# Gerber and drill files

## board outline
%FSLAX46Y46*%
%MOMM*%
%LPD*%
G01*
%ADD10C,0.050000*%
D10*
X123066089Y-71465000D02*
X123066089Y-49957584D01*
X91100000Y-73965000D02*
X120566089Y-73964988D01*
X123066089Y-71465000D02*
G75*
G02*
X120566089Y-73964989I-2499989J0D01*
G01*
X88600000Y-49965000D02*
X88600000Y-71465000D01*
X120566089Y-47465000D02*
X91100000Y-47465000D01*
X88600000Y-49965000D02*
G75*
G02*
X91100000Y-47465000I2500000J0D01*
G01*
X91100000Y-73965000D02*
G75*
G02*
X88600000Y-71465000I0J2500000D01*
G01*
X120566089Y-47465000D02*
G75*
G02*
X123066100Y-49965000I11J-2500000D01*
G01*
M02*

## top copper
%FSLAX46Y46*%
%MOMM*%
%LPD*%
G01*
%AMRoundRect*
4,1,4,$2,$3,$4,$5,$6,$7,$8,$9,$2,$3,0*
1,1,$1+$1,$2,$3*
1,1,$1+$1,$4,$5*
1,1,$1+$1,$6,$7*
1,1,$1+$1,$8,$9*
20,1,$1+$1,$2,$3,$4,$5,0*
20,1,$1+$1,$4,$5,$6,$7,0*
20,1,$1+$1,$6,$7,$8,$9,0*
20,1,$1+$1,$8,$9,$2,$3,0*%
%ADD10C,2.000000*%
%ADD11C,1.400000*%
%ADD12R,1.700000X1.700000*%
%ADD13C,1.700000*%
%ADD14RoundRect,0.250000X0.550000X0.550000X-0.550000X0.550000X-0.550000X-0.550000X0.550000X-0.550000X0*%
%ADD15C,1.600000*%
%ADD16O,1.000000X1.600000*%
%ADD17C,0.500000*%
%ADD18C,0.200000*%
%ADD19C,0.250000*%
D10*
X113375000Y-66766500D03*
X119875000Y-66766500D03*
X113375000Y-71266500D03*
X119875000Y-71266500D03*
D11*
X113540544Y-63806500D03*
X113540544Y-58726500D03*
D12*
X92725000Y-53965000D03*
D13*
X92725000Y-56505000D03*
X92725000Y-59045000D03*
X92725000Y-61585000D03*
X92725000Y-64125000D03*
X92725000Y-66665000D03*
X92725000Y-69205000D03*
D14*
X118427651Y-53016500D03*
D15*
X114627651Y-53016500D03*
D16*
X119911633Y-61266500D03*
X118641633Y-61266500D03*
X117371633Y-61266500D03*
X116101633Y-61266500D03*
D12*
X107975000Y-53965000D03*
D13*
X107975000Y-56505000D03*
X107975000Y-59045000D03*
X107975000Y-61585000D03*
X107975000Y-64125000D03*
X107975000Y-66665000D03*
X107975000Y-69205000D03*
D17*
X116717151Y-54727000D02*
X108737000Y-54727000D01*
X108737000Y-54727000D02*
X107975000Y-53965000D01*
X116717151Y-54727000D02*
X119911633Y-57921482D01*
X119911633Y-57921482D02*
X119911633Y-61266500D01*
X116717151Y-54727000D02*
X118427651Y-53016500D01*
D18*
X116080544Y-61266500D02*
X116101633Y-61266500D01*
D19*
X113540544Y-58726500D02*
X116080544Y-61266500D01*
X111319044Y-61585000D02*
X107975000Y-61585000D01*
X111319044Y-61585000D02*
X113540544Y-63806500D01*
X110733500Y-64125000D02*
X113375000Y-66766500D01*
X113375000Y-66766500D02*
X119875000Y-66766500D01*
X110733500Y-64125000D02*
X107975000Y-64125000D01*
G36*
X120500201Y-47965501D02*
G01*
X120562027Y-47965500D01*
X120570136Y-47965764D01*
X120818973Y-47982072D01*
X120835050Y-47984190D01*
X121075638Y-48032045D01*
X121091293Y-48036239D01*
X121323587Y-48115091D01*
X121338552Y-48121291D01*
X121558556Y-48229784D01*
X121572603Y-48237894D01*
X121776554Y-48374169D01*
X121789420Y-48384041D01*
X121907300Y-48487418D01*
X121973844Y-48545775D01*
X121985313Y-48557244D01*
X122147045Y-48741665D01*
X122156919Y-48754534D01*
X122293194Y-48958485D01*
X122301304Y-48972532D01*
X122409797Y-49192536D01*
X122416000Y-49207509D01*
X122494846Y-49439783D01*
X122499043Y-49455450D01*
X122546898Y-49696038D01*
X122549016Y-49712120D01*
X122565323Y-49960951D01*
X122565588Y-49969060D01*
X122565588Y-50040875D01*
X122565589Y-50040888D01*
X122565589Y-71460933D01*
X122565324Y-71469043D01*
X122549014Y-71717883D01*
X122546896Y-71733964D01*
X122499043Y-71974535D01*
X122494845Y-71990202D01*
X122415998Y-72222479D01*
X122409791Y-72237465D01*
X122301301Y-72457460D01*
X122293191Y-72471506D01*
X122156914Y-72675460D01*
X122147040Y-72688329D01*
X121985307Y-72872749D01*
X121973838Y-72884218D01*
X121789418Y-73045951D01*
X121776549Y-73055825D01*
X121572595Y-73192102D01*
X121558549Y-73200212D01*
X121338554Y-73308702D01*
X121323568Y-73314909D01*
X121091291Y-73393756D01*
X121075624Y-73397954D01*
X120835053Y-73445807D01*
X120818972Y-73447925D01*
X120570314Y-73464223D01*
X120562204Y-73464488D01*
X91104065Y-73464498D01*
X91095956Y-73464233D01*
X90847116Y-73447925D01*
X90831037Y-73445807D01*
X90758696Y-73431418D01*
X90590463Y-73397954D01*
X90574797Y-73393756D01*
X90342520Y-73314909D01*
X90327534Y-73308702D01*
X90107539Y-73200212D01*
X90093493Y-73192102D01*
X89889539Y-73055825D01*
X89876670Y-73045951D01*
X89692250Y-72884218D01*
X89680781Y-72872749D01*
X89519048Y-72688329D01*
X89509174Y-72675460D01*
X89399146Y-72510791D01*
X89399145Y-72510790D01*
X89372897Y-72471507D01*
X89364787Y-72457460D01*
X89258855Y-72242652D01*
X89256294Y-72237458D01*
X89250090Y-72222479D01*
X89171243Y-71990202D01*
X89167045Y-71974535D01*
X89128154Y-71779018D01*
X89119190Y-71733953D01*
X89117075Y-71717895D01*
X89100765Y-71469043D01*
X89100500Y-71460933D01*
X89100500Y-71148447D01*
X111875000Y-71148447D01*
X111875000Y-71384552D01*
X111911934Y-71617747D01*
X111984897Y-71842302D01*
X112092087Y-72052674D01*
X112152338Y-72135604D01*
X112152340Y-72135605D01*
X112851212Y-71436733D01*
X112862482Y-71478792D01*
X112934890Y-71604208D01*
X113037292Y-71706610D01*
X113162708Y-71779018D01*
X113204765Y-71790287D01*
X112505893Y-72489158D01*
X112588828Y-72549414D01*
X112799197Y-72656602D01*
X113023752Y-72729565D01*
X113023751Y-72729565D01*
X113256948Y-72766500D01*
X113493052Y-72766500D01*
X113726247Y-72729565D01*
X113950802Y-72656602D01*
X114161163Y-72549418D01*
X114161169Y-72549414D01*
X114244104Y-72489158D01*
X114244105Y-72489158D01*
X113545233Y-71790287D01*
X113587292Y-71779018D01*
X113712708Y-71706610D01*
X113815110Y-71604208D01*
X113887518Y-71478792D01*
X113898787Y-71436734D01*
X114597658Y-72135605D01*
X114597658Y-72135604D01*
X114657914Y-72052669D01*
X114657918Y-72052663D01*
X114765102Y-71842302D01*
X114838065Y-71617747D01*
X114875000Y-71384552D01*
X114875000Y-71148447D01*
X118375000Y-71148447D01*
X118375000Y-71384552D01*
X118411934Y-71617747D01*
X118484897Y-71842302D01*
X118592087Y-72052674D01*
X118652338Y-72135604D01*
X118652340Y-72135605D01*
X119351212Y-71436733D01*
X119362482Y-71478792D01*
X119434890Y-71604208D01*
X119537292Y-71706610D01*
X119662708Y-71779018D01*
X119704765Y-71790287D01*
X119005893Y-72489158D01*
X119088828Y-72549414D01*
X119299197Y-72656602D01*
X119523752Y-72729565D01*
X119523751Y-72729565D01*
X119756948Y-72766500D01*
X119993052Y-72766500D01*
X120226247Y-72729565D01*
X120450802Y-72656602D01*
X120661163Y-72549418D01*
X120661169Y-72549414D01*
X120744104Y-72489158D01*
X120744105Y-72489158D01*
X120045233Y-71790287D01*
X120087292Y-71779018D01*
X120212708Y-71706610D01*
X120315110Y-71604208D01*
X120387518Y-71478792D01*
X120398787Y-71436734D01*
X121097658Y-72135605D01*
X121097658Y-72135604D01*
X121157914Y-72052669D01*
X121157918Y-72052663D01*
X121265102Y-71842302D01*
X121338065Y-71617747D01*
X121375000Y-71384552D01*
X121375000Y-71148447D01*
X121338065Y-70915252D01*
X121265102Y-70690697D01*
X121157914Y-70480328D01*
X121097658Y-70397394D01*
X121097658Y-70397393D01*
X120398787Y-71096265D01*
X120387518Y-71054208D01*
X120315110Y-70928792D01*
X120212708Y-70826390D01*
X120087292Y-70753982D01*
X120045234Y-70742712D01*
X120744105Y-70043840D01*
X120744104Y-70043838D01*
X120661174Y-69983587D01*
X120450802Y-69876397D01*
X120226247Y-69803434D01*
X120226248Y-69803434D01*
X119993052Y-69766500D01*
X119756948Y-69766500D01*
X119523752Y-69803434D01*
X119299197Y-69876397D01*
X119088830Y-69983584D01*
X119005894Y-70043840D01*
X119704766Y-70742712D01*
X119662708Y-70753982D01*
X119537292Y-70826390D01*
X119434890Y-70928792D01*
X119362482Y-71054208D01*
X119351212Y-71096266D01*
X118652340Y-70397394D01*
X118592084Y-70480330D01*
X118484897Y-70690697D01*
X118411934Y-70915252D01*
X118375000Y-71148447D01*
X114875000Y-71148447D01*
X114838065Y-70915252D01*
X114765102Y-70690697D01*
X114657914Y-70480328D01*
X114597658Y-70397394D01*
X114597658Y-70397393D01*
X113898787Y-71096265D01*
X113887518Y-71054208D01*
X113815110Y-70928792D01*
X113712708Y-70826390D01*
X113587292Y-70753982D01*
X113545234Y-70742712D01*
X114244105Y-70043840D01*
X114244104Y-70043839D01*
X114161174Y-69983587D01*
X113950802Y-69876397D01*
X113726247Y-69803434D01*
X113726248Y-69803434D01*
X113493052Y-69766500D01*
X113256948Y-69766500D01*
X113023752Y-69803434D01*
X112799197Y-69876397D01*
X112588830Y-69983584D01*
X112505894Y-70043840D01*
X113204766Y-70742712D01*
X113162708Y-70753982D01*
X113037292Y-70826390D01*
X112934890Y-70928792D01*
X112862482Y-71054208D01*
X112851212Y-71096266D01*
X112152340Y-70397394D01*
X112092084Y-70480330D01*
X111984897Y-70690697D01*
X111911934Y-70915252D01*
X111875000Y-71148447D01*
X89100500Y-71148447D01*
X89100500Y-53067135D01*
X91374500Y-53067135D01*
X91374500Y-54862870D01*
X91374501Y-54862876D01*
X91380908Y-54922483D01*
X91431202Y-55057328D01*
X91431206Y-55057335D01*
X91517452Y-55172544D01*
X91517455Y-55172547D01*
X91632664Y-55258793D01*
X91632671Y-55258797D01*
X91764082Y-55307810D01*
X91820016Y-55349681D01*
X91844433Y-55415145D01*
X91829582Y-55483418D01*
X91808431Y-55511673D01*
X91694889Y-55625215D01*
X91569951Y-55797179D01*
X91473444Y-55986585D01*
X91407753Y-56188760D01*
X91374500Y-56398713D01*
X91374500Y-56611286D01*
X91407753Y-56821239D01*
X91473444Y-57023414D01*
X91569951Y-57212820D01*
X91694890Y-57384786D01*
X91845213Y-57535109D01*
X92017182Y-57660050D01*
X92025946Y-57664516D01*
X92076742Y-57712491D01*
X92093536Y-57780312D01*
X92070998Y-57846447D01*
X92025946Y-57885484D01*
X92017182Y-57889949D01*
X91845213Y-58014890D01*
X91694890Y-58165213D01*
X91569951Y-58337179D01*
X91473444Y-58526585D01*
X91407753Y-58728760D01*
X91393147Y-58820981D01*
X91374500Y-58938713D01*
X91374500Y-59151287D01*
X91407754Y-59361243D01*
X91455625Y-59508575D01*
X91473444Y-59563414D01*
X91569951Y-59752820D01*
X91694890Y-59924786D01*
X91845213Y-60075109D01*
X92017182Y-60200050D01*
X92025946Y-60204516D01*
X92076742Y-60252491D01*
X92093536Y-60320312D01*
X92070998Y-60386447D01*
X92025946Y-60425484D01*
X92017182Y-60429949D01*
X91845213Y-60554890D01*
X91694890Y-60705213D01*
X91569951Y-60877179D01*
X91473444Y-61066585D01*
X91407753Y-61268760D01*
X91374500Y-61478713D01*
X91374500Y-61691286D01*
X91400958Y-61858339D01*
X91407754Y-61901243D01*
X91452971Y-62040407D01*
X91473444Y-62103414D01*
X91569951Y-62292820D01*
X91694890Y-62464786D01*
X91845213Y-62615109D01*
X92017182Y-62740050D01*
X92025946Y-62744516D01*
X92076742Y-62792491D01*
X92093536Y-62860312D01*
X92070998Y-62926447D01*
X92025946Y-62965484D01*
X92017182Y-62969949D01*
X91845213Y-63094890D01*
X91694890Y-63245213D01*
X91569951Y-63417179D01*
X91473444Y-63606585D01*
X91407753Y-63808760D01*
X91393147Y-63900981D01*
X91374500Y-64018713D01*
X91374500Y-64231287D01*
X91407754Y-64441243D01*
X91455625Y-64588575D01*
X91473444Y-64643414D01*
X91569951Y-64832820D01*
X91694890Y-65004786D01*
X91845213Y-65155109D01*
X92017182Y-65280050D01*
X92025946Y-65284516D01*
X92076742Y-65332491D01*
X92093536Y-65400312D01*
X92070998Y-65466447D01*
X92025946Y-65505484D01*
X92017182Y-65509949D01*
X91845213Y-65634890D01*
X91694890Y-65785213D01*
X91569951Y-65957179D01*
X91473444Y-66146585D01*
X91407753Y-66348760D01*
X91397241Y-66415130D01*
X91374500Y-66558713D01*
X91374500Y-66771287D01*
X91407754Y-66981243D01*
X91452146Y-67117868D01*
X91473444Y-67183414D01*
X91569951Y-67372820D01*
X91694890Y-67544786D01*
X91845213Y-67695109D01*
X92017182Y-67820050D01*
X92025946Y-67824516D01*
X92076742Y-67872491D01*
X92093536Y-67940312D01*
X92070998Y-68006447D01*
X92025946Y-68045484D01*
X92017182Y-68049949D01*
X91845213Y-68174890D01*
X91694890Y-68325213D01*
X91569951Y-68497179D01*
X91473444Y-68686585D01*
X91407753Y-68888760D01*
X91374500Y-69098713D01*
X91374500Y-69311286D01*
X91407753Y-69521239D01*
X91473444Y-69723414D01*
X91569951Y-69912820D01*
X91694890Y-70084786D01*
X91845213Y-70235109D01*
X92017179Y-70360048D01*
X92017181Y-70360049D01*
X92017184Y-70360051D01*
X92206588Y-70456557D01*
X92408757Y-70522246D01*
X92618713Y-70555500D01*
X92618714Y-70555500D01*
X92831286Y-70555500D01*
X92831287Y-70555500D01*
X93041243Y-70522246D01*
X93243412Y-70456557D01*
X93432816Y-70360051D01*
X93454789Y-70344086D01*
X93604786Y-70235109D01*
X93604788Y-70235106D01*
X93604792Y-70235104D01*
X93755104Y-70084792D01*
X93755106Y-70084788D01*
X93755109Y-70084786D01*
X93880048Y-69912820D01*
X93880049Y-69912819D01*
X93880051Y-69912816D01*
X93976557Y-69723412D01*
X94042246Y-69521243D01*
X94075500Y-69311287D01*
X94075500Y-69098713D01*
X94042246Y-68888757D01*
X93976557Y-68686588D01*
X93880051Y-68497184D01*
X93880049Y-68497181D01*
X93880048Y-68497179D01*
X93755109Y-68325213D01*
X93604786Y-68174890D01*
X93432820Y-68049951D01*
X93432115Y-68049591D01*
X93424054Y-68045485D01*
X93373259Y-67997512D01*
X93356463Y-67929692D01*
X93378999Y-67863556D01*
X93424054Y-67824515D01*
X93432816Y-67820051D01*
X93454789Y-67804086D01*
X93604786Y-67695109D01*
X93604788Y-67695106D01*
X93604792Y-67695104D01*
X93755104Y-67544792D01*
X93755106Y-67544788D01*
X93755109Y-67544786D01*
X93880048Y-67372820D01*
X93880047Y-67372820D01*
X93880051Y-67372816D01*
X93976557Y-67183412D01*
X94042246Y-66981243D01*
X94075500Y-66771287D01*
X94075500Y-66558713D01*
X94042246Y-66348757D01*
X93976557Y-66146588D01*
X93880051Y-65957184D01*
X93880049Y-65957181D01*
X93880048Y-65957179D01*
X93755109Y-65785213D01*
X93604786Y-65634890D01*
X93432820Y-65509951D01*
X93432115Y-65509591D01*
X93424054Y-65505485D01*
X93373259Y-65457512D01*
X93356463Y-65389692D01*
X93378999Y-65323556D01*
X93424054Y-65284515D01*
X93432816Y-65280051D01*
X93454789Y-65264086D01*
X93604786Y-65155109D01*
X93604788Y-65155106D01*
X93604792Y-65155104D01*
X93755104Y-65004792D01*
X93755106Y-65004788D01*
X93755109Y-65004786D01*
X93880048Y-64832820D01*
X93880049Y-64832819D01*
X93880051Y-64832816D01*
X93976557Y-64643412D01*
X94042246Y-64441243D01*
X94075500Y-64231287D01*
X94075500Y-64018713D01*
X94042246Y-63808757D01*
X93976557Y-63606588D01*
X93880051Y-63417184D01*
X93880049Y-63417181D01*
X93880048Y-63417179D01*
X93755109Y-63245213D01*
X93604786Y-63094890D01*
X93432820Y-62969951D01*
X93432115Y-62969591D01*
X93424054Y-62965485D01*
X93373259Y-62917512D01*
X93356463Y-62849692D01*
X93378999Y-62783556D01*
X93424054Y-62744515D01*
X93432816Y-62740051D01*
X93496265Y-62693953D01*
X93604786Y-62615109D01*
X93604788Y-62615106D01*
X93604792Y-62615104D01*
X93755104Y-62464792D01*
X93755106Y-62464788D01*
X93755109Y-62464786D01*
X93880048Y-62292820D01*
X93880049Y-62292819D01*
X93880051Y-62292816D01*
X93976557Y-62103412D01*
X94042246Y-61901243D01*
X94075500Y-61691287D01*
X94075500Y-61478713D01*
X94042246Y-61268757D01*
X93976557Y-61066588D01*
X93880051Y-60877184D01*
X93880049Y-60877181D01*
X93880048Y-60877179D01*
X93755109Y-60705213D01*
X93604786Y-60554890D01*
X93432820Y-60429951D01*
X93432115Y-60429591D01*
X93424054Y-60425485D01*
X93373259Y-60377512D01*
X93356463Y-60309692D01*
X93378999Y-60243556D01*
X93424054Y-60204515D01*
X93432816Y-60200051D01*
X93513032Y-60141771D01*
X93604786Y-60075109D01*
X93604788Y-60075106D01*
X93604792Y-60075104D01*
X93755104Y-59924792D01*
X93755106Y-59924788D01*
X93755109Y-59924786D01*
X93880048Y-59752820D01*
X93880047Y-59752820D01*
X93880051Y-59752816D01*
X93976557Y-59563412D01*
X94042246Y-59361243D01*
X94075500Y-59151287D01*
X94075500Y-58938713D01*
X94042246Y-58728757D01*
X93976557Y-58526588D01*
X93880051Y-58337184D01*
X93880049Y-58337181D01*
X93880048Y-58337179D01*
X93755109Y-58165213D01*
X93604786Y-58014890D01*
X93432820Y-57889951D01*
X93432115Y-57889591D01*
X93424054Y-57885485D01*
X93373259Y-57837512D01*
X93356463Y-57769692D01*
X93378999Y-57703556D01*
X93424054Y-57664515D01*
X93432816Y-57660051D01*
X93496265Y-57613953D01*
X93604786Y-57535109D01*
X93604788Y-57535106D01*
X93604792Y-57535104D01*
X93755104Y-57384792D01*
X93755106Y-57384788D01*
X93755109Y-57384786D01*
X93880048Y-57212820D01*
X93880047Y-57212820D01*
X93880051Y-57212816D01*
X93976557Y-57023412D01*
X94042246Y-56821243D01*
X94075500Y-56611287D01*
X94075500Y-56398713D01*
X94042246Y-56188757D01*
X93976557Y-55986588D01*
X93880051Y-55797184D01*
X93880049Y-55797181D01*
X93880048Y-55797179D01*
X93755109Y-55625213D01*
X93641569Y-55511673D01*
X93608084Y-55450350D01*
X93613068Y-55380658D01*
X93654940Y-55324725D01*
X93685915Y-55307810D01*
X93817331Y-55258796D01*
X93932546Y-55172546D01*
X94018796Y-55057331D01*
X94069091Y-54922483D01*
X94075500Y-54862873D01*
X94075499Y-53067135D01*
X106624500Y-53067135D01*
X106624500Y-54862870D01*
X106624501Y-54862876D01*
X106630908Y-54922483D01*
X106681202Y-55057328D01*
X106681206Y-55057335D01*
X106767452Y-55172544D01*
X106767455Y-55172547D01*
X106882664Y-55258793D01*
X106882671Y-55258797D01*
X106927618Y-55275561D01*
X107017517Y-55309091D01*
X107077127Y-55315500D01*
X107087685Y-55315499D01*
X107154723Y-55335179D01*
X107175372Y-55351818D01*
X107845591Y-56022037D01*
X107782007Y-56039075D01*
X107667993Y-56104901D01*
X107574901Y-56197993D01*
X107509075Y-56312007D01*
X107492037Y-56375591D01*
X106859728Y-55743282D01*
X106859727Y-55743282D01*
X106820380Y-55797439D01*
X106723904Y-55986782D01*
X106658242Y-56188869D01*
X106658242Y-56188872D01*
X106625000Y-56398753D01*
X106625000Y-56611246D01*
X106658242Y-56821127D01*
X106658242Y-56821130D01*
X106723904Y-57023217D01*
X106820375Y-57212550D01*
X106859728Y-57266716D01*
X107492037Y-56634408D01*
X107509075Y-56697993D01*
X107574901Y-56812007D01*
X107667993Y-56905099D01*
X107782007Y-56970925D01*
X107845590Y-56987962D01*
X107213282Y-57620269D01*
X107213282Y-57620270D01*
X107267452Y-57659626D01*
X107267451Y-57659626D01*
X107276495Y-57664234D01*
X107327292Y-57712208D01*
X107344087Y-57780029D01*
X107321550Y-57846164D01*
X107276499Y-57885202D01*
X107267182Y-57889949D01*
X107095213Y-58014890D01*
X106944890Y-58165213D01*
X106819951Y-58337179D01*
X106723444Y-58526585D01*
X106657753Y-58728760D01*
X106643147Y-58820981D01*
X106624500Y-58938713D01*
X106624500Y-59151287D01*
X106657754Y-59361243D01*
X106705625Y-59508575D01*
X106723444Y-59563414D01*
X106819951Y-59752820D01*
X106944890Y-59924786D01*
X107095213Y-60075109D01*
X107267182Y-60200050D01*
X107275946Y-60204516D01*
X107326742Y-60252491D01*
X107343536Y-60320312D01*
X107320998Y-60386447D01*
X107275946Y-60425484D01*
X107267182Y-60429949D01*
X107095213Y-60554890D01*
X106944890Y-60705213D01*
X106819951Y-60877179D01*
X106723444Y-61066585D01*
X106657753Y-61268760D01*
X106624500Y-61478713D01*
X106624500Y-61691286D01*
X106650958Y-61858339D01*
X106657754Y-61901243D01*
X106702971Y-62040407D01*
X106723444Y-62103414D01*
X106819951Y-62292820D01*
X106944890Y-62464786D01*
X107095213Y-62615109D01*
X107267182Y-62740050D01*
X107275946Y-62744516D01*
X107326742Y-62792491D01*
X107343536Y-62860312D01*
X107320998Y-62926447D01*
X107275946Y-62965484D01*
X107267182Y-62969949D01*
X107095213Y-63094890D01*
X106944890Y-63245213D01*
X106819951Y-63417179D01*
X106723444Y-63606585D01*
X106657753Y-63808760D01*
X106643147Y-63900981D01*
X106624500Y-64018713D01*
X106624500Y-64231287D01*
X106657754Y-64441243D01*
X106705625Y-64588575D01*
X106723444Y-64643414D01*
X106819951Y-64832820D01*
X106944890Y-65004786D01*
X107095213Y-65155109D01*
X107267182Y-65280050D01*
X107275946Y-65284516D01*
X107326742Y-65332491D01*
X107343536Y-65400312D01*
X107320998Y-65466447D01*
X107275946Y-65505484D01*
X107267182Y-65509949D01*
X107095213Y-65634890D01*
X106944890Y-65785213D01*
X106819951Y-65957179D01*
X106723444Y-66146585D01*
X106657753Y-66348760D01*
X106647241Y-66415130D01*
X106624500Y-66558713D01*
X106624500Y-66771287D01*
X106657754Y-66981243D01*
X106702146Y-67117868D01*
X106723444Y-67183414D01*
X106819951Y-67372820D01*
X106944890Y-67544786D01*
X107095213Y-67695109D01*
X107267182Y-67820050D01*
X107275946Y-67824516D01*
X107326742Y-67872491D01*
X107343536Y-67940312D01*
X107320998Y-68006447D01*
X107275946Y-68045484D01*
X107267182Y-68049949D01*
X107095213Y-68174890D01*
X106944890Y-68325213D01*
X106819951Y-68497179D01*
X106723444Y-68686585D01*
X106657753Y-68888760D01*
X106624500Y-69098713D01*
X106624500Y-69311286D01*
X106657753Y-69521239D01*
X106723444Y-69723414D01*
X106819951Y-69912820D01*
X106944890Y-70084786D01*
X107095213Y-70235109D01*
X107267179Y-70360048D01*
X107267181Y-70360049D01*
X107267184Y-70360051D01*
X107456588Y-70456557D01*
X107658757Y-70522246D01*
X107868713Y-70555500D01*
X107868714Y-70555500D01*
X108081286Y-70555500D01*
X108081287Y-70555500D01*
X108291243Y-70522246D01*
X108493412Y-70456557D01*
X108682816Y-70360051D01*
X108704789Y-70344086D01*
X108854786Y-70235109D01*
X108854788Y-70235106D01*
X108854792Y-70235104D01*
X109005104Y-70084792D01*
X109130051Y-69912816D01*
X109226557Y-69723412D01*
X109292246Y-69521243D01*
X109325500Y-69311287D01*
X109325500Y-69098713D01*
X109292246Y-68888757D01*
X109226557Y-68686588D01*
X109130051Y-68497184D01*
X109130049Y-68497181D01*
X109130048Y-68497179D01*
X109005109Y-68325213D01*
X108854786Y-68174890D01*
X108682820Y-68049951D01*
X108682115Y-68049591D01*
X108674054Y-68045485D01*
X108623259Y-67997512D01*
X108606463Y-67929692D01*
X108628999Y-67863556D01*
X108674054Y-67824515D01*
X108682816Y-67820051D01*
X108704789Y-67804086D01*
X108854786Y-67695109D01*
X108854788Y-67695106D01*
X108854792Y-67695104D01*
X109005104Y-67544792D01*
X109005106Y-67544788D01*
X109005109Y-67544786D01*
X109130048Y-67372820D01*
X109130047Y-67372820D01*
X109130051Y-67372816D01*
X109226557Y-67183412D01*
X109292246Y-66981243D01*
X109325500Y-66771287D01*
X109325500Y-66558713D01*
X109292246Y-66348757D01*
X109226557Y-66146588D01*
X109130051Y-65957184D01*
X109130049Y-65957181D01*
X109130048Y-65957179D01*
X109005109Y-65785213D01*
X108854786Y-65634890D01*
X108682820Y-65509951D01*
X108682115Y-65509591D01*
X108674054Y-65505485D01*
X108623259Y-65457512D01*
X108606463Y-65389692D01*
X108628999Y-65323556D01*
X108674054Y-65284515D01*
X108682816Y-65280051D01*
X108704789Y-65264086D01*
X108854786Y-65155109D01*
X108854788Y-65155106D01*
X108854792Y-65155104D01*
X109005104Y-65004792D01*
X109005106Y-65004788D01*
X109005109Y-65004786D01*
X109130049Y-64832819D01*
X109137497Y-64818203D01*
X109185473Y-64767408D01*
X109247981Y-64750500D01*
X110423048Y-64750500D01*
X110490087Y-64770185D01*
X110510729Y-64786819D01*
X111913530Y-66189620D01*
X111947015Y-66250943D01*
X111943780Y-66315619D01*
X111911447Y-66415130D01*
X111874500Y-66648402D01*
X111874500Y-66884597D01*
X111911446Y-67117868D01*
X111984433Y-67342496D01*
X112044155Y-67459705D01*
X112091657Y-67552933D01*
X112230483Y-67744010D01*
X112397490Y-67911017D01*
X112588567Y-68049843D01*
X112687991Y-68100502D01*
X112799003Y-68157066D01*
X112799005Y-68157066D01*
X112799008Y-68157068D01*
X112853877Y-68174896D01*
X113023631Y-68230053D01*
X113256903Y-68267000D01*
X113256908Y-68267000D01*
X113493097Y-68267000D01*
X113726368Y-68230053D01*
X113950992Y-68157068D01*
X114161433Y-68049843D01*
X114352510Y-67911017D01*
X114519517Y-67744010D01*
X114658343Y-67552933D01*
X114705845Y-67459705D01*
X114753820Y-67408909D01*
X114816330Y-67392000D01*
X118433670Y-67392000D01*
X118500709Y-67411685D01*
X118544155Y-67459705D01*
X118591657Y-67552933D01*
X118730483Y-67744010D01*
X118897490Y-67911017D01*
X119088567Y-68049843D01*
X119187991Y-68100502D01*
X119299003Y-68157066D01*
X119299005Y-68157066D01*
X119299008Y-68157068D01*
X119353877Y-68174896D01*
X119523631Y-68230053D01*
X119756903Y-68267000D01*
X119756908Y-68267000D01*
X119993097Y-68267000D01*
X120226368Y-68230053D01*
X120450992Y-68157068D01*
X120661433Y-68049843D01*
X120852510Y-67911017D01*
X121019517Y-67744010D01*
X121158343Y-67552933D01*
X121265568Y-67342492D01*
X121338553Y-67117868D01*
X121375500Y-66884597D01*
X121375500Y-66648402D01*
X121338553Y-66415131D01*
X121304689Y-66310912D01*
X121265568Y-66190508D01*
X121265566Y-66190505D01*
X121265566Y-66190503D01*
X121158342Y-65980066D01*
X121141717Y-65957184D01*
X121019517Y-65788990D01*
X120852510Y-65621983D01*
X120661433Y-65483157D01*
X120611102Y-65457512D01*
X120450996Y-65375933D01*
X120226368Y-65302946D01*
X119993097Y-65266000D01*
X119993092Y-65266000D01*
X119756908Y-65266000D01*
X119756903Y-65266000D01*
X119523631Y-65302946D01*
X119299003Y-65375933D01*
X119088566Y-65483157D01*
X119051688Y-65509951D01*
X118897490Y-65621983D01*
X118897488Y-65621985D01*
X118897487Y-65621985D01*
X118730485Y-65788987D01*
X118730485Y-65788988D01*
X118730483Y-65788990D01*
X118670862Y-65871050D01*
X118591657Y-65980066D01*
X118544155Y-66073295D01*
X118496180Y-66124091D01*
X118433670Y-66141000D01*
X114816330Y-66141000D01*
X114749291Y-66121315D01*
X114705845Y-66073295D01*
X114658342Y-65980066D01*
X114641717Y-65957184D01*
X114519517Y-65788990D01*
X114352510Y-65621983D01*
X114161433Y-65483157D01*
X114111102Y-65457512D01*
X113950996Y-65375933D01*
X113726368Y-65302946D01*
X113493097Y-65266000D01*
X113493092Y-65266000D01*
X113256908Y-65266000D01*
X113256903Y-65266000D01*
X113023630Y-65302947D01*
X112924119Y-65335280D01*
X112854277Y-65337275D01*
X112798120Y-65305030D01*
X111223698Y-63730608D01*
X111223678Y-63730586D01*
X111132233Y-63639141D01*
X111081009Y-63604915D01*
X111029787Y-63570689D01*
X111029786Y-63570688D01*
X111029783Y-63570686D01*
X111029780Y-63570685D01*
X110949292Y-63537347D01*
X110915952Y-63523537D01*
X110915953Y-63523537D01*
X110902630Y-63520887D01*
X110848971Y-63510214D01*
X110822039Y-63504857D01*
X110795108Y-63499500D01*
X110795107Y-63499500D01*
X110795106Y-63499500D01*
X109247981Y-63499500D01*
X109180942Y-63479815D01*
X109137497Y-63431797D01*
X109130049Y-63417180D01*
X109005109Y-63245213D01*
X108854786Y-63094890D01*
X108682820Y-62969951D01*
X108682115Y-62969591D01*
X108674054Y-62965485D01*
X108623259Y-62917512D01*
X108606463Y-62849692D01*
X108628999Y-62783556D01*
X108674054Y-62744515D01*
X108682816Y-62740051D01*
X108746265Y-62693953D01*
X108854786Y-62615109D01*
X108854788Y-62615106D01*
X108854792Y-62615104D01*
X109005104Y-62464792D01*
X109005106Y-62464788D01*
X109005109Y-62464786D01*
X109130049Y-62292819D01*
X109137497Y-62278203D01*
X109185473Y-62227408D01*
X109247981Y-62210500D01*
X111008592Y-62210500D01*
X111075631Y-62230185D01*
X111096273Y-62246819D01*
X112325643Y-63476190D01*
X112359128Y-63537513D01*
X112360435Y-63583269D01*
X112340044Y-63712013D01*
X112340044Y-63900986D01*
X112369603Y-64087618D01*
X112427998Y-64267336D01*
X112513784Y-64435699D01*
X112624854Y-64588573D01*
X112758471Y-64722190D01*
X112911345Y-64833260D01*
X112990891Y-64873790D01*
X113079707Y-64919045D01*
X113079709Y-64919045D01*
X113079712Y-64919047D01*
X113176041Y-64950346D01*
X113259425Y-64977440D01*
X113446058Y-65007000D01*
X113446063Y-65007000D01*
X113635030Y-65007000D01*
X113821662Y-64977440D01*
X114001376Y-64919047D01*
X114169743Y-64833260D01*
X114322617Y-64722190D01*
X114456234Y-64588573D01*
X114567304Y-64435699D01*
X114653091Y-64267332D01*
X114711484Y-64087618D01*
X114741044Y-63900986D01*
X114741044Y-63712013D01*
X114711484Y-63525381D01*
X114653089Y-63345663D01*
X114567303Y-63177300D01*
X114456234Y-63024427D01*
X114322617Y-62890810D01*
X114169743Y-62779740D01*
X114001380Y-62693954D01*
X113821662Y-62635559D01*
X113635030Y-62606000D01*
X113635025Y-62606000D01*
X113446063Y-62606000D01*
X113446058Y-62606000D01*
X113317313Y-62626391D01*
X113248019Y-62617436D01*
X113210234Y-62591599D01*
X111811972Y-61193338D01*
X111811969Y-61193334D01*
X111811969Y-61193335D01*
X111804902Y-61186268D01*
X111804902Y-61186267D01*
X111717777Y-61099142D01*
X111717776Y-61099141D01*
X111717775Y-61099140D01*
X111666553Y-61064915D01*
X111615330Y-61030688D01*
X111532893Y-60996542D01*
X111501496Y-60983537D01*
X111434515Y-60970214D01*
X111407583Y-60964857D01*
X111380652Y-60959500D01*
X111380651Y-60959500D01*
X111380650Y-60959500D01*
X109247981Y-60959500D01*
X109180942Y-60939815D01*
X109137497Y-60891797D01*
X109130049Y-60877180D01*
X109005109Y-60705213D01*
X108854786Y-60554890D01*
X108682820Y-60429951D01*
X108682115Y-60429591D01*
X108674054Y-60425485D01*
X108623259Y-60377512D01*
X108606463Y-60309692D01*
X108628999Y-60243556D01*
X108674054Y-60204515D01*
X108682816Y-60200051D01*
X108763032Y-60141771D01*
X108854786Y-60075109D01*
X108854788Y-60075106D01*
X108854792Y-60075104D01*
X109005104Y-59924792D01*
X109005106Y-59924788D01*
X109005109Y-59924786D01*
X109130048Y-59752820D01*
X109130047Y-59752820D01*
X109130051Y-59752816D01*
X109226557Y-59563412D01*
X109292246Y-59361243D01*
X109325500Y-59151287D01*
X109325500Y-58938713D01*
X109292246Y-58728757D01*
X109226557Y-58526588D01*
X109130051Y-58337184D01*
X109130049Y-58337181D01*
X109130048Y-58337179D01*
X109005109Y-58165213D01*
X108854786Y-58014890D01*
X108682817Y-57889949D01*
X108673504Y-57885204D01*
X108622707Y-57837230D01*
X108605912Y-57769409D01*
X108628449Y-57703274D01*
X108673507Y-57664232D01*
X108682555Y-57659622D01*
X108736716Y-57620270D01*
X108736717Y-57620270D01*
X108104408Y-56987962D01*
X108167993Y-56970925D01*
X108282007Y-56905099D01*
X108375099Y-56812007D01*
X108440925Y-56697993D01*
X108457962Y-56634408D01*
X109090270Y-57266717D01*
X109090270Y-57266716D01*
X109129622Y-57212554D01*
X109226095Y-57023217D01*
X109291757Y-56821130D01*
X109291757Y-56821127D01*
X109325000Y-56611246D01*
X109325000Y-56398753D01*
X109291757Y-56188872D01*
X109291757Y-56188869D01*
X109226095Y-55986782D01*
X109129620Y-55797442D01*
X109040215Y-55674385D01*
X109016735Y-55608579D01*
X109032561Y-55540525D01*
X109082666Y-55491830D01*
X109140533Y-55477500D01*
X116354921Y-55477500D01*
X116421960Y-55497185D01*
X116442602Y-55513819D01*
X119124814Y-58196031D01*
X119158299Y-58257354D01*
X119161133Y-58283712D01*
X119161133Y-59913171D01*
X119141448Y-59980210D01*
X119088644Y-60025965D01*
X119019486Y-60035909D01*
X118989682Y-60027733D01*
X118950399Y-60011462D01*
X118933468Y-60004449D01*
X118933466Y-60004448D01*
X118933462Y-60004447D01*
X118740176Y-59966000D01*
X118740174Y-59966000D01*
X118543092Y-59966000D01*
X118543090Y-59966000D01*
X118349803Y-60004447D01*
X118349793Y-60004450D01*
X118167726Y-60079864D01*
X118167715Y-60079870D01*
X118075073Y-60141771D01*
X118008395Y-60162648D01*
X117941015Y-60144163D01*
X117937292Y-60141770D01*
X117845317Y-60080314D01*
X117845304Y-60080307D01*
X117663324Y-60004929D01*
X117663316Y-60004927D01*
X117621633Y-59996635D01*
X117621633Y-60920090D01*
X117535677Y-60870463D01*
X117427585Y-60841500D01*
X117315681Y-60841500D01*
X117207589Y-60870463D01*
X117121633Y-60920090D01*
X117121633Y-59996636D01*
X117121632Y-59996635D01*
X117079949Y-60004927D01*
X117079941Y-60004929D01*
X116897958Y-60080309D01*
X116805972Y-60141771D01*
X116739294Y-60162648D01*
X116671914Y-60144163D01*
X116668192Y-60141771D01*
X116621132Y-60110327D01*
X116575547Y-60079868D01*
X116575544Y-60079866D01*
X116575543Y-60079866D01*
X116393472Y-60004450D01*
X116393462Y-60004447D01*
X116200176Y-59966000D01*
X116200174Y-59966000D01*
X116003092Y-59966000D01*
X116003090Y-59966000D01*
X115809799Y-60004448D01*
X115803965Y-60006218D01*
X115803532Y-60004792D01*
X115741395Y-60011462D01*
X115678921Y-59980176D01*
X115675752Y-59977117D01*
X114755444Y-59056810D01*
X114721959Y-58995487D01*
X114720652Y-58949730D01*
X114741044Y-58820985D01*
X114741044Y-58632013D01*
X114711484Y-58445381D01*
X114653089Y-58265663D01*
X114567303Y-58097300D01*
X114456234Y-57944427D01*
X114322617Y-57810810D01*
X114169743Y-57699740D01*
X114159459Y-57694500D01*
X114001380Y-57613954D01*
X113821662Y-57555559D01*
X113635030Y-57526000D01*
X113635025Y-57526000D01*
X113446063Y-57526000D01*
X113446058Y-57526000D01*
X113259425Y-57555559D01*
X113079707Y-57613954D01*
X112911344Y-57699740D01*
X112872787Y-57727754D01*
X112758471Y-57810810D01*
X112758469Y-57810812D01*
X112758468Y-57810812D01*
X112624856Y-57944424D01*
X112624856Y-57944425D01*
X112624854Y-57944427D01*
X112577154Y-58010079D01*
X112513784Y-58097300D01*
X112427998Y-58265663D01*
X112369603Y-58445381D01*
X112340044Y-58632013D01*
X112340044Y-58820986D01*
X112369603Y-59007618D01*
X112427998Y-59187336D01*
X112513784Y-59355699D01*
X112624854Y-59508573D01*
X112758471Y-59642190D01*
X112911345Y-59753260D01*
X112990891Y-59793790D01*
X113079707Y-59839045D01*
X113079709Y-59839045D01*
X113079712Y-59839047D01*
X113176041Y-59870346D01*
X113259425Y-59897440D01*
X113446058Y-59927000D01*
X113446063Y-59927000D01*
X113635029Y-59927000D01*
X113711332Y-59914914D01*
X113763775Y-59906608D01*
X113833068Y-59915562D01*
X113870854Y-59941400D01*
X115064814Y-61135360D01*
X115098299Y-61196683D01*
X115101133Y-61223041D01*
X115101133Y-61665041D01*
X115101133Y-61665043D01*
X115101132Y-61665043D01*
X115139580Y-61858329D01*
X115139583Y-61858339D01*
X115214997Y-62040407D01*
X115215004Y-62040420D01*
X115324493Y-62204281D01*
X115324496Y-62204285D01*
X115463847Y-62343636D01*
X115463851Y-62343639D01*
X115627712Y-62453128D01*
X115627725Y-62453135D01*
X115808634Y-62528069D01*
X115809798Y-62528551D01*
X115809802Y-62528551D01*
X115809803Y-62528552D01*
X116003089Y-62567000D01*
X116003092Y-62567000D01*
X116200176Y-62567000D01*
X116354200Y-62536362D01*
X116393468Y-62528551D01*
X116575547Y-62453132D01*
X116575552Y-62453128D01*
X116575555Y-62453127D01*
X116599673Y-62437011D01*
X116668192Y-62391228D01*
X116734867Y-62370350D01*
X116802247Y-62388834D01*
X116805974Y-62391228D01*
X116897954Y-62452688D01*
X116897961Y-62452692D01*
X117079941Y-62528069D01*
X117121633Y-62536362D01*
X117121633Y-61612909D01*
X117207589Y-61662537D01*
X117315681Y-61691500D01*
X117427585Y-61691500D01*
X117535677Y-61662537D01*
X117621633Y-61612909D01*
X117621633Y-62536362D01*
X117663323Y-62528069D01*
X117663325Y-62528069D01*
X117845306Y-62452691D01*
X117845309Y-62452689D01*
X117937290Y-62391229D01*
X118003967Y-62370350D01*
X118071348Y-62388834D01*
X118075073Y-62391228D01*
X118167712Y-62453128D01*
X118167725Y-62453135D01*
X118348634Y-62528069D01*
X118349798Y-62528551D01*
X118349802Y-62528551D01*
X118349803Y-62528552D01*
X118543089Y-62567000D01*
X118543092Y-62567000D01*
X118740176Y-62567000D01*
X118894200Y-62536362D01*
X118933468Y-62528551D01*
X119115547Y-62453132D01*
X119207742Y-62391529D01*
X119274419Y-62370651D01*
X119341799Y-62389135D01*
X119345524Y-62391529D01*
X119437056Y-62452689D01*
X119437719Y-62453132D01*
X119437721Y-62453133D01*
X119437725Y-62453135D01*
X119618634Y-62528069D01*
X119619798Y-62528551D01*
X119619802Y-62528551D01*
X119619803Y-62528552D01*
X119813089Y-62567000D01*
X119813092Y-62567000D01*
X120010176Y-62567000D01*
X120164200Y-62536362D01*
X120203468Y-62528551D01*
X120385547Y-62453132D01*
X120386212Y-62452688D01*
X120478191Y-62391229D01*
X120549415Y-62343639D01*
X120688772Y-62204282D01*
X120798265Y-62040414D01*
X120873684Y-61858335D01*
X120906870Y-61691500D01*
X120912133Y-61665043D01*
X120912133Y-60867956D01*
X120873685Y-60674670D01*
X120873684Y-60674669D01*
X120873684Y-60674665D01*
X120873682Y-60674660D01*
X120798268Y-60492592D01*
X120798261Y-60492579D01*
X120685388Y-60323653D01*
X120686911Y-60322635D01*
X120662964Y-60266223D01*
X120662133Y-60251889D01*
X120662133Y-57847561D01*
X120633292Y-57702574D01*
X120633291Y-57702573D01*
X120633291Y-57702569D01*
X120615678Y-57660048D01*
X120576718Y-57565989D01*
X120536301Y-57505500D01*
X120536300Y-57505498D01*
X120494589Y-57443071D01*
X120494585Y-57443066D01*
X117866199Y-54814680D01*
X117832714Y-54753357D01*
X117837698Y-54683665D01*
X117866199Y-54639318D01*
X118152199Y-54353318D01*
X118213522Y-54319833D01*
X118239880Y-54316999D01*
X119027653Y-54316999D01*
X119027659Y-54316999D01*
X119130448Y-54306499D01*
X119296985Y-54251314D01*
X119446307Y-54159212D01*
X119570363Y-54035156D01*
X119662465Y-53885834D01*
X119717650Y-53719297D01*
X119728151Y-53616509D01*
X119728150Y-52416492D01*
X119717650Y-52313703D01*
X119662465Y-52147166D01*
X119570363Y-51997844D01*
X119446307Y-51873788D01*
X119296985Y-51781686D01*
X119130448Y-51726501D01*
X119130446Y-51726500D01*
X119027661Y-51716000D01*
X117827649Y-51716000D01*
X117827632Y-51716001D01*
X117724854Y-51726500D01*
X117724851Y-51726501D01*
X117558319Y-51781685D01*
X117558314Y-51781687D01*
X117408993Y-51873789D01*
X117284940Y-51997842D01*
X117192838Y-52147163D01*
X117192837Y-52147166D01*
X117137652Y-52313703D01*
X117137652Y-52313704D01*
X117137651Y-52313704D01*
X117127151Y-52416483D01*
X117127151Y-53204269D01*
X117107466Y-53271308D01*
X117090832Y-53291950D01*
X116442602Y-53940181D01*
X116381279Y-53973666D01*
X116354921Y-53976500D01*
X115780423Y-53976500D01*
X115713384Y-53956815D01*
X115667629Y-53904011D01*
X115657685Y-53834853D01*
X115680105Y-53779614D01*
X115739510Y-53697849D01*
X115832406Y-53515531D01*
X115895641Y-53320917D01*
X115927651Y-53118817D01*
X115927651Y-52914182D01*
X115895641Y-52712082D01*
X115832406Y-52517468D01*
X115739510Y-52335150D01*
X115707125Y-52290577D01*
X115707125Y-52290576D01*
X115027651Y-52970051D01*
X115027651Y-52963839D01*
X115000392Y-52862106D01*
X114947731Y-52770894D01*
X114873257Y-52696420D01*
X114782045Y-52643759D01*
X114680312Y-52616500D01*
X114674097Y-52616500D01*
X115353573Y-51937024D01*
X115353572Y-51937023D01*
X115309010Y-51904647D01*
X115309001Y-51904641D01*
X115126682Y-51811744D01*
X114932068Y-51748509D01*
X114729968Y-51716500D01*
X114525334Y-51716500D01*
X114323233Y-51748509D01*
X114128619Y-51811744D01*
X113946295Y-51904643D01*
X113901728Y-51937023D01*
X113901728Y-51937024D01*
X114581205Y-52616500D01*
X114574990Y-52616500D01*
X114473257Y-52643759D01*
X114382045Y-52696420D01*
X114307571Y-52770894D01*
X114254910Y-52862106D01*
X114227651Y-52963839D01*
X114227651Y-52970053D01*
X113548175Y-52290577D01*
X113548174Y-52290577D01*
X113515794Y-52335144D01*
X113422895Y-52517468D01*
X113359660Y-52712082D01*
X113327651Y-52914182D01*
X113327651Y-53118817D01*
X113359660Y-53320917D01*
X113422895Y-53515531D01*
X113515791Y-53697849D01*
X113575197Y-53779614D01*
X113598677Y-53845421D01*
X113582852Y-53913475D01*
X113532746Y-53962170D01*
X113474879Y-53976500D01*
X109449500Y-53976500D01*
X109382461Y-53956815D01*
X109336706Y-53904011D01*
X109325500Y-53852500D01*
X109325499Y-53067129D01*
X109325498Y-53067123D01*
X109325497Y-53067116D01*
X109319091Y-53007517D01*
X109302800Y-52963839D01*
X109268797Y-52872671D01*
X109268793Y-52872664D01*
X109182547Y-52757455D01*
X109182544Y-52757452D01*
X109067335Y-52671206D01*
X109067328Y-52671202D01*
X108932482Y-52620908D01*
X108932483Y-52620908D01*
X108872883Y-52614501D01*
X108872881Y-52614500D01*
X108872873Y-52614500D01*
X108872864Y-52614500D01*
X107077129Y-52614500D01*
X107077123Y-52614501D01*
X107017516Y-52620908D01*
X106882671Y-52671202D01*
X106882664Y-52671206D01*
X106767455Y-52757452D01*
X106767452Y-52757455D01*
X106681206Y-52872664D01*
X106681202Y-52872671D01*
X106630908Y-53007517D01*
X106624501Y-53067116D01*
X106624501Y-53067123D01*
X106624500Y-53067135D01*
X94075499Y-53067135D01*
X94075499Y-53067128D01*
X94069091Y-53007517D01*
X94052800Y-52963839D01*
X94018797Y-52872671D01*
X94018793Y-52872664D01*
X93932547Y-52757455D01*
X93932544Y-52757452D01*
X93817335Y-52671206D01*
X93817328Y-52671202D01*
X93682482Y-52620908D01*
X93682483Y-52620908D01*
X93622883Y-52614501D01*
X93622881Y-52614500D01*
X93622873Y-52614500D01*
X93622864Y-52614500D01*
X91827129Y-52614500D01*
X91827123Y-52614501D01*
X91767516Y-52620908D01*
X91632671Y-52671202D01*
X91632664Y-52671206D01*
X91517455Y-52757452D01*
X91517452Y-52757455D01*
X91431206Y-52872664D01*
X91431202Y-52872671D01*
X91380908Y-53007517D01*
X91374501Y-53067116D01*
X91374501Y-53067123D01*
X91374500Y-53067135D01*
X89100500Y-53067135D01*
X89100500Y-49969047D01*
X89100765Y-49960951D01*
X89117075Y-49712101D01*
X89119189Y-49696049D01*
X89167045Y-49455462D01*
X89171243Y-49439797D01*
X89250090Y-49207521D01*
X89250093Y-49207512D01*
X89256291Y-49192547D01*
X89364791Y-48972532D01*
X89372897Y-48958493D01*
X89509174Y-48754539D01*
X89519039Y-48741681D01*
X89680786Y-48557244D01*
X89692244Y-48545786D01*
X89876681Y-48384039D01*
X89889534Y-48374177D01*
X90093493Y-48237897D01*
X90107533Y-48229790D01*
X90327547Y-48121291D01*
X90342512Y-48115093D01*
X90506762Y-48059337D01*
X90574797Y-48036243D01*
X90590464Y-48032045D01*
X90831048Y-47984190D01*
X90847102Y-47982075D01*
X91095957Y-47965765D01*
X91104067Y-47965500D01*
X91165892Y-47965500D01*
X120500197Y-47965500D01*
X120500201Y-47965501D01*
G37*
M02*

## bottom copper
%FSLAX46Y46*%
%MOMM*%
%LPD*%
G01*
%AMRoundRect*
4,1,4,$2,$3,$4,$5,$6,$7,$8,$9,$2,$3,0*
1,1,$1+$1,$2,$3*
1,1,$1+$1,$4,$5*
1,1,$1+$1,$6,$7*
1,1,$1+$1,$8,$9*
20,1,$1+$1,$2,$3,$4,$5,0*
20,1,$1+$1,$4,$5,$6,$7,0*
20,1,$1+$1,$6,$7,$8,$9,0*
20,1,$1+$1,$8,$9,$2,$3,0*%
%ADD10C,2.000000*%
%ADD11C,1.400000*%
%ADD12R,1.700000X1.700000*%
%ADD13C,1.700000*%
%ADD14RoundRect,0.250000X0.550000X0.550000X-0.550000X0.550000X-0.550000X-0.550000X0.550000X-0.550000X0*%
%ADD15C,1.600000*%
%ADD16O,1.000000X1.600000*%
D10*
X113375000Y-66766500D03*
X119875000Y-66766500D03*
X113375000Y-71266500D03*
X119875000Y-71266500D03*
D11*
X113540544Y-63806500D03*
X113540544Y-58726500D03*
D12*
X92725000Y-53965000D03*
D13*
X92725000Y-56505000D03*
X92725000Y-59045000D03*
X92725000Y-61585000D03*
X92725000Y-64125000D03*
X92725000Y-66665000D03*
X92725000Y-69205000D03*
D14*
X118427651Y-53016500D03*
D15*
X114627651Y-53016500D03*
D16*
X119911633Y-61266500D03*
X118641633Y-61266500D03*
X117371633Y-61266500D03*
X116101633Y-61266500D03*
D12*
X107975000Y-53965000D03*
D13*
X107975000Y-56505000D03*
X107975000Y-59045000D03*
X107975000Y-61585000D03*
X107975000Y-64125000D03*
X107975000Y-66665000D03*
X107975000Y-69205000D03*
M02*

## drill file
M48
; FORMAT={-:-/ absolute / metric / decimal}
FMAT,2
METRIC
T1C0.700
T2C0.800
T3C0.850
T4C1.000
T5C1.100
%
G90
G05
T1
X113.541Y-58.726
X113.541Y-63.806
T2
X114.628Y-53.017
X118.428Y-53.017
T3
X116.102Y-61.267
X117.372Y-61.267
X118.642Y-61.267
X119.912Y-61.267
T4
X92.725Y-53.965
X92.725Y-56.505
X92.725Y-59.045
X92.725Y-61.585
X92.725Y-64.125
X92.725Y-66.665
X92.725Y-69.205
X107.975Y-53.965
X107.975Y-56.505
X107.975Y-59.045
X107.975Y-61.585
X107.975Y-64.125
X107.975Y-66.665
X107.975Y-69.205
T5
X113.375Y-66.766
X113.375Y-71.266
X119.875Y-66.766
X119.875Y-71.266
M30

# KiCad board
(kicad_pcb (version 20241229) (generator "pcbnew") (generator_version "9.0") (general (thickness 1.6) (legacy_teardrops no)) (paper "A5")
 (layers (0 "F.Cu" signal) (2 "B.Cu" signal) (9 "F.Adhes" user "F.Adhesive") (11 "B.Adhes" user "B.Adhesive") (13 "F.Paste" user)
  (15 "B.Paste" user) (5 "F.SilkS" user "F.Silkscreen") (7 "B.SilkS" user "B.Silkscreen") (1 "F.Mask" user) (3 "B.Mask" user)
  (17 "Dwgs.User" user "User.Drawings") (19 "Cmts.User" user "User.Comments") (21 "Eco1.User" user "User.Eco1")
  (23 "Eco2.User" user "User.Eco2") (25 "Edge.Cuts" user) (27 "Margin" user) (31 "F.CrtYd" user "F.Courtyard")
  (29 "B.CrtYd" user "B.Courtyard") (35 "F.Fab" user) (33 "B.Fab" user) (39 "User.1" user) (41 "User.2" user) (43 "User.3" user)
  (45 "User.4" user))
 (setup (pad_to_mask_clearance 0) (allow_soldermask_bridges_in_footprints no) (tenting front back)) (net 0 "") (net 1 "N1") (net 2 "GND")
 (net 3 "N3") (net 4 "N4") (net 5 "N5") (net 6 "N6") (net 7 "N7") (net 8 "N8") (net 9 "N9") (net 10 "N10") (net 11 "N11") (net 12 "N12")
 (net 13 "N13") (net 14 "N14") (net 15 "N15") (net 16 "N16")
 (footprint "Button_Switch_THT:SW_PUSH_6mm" (layer "F.Cu") (at 113.375 66.7665)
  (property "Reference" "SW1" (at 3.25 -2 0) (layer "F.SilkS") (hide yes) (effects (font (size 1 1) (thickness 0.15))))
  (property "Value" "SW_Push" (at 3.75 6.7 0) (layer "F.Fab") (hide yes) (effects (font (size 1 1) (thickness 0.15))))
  (pad "1" thru_hole circle (at 0 0 90) (size 2 2) (drill 1.1) (layers "*.Cu" "*.Mask") (remove_unused_layers no) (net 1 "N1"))
  (pad "1" thru_hole circle (at 6.5 0 90) (size 2 2) (drill 1.1) (layers "*.Cu" "*.Mask") (remove_unused_layers no) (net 1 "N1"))
  (pad "2" thru_hole circle (at 0 4.5 90) (size 2 2) (drill 1.1) (layers "*.Cu" "*.Mask") (remove_unused_layers no) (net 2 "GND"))
  (pad "2" thru_hole circle (at 6.5 4.5 90) (size 2 2) (drill 1.1) (layers "*.Cu" "*.Mask") (remove_unused_layers no) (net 2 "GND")))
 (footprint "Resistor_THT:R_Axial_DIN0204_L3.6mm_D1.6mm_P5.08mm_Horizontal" (layer "F.Cu") (at 113.540544 63.8065 90)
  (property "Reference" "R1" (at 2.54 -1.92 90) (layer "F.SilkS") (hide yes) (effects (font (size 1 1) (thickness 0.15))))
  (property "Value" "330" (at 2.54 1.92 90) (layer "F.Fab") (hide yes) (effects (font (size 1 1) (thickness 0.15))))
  (pad "1" thru_hole circle (at 0 0 90) (size 1.4 1.4) (drill 0.7) (layers "*.Cu" "*.Mask") (remove_unused_layers no) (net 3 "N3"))
  (pad "2" thru_hole circle (at 5.08 0 90) (size 1.4 1.4) (drill 0.7) (layers "*.Cu" "*.Mask") (remove_unused_layers no) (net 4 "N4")))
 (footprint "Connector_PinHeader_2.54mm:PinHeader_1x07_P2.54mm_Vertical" (layer "F.Cu") (at 92.725 53.965)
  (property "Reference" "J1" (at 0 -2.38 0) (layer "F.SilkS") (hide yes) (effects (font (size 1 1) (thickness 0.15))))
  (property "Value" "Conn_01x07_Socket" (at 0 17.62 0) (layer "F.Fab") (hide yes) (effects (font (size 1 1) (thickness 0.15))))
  (pad "1" thru_hole rect (at 0 0) (size 1.7 1.7) (drill 1) (layers "*.Cu" "*.Mask") (remove_unused_layers no) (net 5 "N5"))
  (pad "2" thru_hole circle (at 0 2.54) (size 1.7 1.7) (drill 1) (layers "*.Cu" "*.Mask") (remove_unused_layers no) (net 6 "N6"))
  (pad "3" thru_hole circle (at 0 5.08) (size 1.7 1.7) (drill 1) (layers "*.Cu" "*.Mask") (remove_unused_layers no) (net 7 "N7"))
  (pad "4" thru_hole circle (at 0 7.62) (size 1.7 1.7) (drill 1) (layers "*.Cu" "*.Mask") (remove_unused_layers no) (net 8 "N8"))
  (pad "5" thru_hole circle (at 0 10.16) (size 1.7 1.7) (drill 1) (layers "*.Cu" "*.Mask") (remove_unused_layers no) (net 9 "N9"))
  (pad "6" thru_hole circle (at 0 12.7) (size 1.7 1.7) (drill 1) (layers "*.Cu" "*.Mask") (remove_unused_layers no) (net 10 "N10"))
  (pad "7" thru_hole circle (at 0 15.24) (size 1.7 1.7) (drill 1) (layers "*.Cu" "*.Mask") (remove_unused_layers no) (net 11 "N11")))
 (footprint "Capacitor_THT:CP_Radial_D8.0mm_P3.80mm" (layer "F.Cu") (at 118.427651 53.0165 180)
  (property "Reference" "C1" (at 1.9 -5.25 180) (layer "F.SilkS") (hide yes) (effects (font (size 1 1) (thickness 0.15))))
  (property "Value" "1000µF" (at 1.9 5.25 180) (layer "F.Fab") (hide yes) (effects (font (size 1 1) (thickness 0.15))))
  (pad "1" thru_hole roundrect (at 0 0 180) (size 1.6 1.6) (drill 0.8) (layers "*.Cu" "*.Mask") (remove_unused_layers no)
   (roundrect_rratio 0.15625) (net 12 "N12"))
  (pad "2" thru_hole circle (at 3.8 0 180) (size 1.6 1.6) (drill 0.8) (layers "*.Cu" "*.Mask") (remove_unused_layers no) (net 2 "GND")))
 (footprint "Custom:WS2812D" (layer "F.Cu") (at 118.006633 61.2665 180)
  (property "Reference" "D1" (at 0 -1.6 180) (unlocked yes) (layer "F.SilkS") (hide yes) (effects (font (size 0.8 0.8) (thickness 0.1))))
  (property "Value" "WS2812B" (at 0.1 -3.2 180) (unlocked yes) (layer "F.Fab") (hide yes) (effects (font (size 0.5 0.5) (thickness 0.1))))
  (pad "1" thru_hole oval (at -1.905 0 180) (size 1 1.6) (drill 0.85) (layers "*.Cu" "*.Mask") (remove_unused_layers no) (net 12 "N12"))
  (pad "2" thru_hole oval (at -0.635 0 180) (size 1 1.6) (drill 0.85) (layers "*.Cu" "*.Mask") (remove_unused_layers no) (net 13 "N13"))
  (pad "3" thru_hole oval (at 0.635 0 180) (size 1 1.6) (drill 0.85) (layers "*.Cu" "*.Mask") (remove_unused_layers no) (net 2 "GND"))
  (pad "4" thru_hole oval (at 1.905 0 180) (size 1 1.6) (drill 0.85) (layers "*.Cu" "*.Mask") (remove_unused_layers no) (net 4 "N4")))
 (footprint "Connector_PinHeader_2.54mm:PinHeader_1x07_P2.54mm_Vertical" (layer "F.Cu") (at 107.975 53.965)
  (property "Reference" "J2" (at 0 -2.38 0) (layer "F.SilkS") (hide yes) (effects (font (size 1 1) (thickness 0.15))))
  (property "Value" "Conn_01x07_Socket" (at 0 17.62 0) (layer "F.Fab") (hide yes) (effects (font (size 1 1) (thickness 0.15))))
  (pad "1" thru_hole rect (at 0 0) (size 1.7 1.7) (drill 1) (layers "*.Cu" "*.Mask") (remove_unused_layers no) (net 12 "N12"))
  (pad "2" thru_hole circle (at 0 2.54) (size 1.7 1.7) (drill 1) (layers "*.Cu" "*.Mask") (remove_unused_layers no) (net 2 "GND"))
  (pad "3" thru_hole circle (at 0 5.08) (size 1.7 1.7) (drill 1) (layers "*.Cu" "*.Mask") (remove_unused_layers no) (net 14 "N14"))
  (pad "4" thru_hole circle (at 0 7.62) (size 1.7 1.7) (drill 1) (layers "*.Cu" "*.Mask") (remove_unused_layers no) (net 3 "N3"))
  (pad "5" thru_hole circle (at 0 10.16) (size 1.7 1.7) (drill 1) (layers "*.Cu" "*.Mask") (remove_unused_layers no) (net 1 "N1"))
  (pad "6" thru_hole circle (at 0 12.7) (size 1.7 1.7) (drill 1) (layers "*.Cu" "*.Mask") (remove_unused_layers no) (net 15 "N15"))
  (pad "7" thru_hole circle (at 0 15.24) (size 1.7 1.7) (drill 1) (layers "*.Cu" "*.Mask") (remove_unused_layers no) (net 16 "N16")))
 (gr_line (start 123.066089 71.465) (end 123.066089 49.957584) (stroke (width 0.05) (type default)) (layer "Edge.Cuts"))
 (gr_line (start 91.1 73.965) (end 120.566089 73.964988) (stroke (width 0.05) (type default)) (layer "Edge.Cuts"))
 (gr_arc (start 123.066089 71.465) (mid 122.333856 73.232767) (end 120.566089 73.965) (stroke (width 0.05) (type default))
  (layer "Edge.Cuts"))
 (gr_line (start 88.6 49.965) (end 88.6 71.465) (stroke (width 0.05) (type default)) (layer "Edge.Cuts"))
 (gr_line (start 120.566089 47.465) (end 91.1 47.465) (stroke (width 0.05) (type default)) (layer "Edge.Cuts"))
 (gr_arc (start 88.6 49.965) (mid 89.332233 48.197233) (end 91.1 47.465) (stroke (width 0.05) (type default)) (layer "Edge.Cuts"))
 (gr_arc (start 91.1 73.965) (mid 89.332233 73.232767) (end 88.6 71.465) (stroke (width 0.05) (type default)) (layer "Edge.Cuts"))
 (gr_arc (start 120.566089 47.465) (mid 122.333863 48.197229) (end 123.066089 49.965) (stroke (width 0.05) (type default))
  (layer "Edge.Cuts"))
 (segment (start 116.717151 54.727) (end 108.737 54.727) (width 0.5) (layer "F.Cu") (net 12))
 (segment (start 108.737 54.727) (end 107.975 53.965) (width 0.5) (layer "F.Cu") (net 12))
 (segment (start 116.717151 54.727) (end 119.911633 57.921482) (width 0.5) (layer "F.Cu") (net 12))
 (segment (start 119.911633 57.921482) (end 119.911633 61.2665) (width 0.5) (layer "F.Cu") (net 12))
 (segment (start 116.717151 54.727) (end 118.427651 53.0165) (width 0.5) (layer "F.Cu") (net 12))
 (segment (start 116.080544 61.2665) (end 116.101633 61.2665) (width 0.2) (layer "F.Cu") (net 4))
 (segment (start 113.540544 58.7265) (end 116.080544 61.2665) (width 0.25) (layer "F.Cu") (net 4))
 (segment (start 111.319044 61.585) (end 107.975 61.585) (width 0.25) (layer "F.Cu") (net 3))
 (segment (start 111.319044 61.585) (end 113.540544 63.8065) (width 0.25) (layer "F.Cu") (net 3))
 (segment (start 110.7335 64.125) (end 113.375 66.7665) (width 0.25) (layer "F.Cu") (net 1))
 (segment (start 113.375 66.7665) (end 119.875 66.7665) (width 0.25) (layer "F.Cu") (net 1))
 (segment (start 110.7335 64.125) (end 107.975 64.125) (width 0.25) (layer "F.Cu") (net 1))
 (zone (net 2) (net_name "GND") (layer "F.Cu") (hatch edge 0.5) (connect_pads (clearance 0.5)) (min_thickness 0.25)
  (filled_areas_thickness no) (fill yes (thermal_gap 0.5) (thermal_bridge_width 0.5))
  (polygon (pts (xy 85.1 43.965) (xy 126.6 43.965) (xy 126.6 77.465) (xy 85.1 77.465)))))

